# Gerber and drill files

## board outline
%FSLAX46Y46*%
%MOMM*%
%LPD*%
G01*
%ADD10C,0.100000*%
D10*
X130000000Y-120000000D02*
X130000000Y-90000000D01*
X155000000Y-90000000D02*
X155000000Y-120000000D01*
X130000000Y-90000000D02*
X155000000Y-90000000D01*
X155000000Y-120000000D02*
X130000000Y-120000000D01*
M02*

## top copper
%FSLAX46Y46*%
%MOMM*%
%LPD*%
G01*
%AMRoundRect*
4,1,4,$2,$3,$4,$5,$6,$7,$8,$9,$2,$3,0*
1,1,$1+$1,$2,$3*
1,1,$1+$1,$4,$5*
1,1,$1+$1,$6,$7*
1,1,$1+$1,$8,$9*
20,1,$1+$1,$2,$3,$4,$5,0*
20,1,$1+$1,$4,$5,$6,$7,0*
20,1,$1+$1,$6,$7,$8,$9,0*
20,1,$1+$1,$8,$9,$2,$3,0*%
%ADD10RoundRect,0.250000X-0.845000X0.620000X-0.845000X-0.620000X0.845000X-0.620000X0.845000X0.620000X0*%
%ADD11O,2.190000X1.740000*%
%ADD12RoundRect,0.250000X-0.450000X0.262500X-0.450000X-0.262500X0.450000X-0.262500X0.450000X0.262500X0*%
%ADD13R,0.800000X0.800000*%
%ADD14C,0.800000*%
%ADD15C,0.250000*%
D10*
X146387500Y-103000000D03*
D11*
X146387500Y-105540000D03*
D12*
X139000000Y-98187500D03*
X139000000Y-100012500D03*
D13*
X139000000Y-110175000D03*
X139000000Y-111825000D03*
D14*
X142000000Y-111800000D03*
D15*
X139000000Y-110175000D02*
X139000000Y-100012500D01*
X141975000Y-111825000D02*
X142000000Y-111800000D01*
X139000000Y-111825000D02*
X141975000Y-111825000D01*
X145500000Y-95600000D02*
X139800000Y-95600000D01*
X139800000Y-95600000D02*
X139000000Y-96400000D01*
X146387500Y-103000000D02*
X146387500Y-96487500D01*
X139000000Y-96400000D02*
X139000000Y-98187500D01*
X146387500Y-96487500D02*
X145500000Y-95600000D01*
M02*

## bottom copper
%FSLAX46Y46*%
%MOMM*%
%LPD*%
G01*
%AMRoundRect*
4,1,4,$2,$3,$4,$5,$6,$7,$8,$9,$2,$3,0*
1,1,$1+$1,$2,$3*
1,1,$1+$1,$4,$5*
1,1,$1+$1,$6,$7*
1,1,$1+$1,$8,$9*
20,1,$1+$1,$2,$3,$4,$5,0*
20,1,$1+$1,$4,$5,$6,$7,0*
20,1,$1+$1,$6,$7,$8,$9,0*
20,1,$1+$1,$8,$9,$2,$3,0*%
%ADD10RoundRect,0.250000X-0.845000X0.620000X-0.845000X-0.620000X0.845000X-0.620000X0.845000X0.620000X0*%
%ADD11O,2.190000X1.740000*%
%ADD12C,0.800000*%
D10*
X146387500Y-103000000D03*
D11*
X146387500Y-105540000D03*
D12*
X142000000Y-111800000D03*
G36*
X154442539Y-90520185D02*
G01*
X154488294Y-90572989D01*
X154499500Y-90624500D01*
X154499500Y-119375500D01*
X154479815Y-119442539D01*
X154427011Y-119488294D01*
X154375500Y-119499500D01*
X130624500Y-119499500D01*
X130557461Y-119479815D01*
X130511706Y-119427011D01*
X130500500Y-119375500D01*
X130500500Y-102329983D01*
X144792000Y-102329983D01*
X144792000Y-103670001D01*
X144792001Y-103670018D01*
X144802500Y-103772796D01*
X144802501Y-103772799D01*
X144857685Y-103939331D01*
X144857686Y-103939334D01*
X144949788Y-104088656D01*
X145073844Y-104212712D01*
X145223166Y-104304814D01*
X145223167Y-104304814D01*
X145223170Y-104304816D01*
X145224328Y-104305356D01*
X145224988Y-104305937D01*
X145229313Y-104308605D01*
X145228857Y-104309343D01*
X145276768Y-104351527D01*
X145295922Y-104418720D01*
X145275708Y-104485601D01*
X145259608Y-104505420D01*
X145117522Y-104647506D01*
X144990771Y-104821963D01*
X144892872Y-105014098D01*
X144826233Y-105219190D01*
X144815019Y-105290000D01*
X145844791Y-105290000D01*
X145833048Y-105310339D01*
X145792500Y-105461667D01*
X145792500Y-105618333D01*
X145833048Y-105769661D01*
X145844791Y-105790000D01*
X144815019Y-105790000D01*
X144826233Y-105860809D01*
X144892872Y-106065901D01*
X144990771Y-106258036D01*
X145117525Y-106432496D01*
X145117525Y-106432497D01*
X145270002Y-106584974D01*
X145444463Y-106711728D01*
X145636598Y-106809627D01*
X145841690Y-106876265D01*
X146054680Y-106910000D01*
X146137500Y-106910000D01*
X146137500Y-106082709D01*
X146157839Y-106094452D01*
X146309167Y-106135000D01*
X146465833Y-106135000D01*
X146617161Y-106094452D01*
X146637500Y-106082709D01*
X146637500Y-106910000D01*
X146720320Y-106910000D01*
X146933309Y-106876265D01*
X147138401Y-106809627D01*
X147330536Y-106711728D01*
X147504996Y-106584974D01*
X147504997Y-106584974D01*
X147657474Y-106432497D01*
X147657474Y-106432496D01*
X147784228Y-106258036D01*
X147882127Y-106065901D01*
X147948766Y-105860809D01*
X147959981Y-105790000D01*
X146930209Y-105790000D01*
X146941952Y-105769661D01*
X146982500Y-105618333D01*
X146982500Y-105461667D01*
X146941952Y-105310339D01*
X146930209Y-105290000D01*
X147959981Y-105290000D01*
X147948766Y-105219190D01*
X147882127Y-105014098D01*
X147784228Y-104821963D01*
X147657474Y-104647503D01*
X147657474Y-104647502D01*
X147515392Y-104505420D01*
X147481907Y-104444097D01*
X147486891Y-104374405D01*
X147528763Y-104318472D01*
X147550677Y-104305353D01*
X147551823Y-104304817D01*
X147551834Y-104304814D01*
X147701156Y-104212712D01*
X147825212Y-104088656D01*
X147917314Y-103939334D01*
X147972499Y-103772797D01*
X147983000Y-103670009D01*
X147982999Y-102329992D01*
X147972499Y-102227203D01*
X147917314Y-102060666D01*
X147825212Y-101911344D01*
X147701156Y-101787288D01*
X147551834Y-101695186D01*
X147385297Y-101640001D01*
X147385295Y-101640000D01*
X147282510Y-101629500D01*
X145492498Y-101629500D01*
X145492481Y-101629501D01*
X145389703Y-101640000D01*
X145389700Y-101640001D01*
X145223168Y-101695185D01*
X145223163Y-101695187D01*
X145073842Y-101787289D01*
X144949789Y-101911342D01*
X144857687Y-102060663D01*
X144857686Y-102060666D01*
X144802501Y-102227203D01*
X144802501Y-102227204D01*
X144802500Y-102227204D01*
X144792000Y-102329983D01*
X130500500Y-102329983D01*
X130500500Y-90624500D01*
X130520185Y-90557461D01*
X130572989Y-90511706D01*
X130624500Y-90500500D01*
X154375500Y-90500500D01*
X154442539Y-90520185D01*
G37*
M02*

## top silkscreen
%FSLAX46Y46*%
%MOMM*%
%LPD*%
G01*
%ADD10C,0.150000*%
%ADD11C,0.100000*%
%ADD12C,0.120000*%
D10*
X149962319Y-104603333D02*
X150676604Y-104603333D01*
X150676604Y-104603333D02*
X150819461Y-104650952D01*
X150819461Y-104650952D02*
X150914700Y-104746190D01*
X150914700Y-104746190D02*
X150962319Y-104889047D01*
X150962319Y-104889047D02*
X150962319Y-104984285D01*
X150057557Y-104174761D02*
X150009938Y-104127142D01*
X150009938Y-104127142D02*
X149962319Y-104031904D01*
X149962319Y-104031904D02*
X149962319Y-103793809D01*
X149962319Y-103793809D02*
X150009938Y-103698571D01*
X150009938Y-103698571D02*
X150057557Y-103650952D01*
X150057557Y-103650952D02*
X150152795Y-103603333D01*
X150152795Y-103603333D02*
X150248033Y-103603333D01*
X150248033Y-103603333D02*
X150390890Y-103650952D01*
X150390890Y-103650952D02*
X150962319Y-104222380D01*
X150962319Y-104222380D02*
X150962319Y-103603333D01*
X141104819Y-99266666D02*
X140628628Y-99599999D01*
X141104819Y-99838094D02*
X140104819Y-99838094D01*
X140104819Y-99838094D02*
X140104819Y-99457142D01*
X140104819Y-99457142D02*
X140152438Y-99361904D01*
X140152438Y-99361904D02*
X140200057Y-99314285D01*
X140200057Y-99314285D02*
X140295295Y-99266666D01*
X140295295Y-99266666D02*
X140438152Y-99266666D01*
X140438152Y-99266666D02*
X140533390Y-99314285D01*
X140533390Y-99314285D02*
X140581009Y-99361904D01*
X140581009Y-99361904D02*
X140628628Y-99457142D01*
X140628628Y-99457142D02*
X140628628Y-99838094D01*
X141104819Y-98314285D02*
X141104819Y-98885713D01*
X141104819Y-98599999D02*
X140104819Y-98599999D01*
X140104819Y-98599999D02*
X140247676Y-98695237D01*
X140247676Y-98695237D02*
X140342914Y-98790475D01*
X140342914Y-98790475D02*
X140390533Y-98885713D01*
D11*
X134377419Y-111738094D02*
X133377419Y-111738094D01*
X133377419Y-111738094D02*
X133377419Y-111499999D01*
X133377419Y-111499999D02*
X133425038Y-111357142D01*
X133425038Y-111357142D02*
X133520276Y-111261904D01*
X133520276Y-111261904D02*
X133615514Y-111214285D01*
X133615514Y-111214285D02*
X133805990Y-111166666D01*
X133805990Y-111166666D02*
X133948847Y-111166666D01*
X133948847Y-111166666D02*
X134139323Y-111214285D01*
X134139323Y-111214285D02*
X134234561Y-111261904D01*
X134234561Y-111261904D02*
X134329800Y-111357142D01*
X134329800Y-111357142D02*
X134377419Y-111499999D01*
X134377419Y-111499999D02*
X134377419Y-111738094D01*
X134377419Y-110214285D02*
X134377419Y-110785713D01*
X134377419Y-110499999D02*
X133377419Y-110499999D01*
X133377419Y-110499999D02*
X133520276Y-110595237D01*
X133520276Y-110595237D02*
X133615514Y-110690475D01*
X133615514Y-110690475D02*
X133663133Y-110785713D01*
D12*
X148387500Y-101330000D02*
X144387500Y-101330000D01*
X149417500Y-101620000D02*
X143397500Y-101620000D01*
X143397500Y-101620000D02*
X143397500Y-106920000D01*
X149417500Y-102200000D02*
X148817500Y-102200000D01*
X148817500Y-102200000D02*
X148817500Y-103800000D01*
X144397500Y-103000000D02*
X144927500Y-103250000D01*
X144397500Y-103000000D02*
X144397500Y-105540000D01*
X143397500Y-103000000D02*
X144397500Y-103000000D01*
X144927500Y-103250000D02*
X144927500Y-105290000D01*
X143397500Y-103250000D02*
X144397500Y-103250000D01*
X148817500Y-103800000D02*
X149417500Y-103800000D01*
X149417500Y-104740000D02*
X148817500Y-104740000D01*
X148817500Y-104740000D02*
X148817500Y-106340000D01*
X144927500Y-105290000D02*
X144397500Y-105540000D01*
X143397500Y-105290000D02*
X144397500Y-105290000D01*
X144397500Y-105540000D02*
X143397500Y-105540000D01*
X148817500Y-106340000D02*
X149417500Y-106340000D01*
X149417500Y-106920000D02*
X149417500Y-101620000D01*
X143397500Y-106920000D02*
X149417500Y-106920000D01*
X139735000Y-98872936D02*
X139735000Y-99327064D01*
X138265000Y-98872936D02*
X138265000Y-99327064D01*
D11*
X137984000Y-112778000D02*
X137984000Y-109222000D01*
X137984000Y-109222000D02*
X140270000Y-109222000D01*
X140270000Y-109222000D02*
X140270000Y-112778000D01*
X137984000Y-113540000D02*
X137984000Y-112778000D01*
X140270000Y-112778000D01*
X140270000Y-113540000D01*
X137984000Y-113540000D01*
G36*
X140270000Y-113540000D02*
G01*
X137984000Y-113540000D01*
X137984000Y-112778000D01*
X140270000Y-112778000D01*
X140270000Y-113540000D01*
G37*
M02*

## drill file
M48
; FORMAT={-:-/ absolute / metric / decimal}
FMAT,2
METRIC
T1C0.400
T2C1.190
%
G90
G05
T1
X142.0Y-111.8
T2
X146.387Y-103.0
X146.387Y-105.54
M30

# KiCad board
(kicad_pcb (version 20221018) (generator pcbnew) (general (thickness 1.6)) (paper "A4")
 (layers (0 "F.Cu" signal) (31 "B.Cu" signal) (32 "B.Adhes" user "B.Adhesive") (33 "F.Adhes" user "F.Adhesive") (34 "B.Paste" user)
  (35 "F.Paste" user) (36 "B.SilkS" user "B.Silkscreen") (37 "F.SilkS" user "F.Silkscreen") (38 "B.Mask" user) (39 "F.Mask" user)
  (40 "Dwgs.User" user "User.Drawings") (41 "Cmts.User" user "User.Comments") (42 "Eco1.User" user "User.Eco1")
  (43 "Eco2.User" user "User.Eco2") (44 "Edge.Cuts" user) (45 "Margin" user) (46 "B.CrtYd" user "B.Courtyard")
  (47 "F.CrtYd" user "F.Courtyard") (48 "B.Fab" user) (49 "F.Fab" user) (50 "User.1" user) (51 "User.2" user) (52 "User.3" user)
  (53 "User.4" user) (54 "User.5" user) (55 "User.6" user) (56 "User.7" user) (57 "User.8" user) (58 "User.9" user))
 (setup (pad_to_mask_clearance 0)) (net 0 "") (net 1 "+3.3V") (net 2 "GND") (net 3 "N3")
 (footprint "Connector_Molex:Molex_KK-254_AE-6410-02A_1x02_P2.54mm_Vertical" (layer "F.Cu") (at 146.3875 103 -90)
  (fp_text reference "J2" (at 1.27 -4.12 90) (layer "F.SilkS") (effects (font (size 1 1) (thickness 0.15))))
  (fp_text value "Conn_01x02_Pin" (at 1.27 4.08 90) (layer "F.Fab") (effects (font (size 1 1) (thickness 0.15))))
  (fp_line (start -1.67 -2) (end -1.67 2) (stroke (width 0.12) (type solid)) (layer "F.SilkS"))
  (fp_line (start -1.38 -3.03) (end -1.38 2.99) (stroke (width 0.12) (type solid)) (layer "F.SilkS"))
  (fp_line (start -1.38 2.99) (end 3.92 2.99) (stroke (width 0.12) (type solid)) (layer "F.SilkS"))
  (fp_line (start -0.8 -3.03) (end -0.8 -2.43) (stroke (width 0.12) (type solid)) (layer "F.SilkS"))
  (fp_line (start -0.8 -2.43) (end 0.8 -2.43) (stroke (width 0.12) (type solid)) (layer "F.SilkS"))
  (fp_line (start 0 1.99) (end 0.25 1.46) (stroke (width 0.12) (type solid)) (layer "F.SilkS"))
  (fp_line (start 0 1.99) (end 2.54 1.99) (stroke (width 0.12) (type solid)) (layer "F.SilkS"))
  (fp_line (start 0 2.99) (end 0 1.99) (stroke (width 0.12) (type solid)) (layer "F.SilkS"))
  (fp_line (start 0.25 1.46) (end 2.29 1.46) (stroke (width 0.12) (type solid)) (layer "F.SilkS"))
  (fp_line (start 0.25 2.99) (end 0.25 1.99) (stroke (width 0.12) (type solid)) (layer "F.SilkS"))
  (fp_line (start 0.8 -2.43) (end 0.8 -3.03) (stroke (width 0.12) (type solid)) (layer "F.SilkS"))
  (fp_line (start 1.74 -3.03) (end 1.74 -2.43) (stroke (width 0.12) (type solid)) (layer "F.SilkS"))
  (fp_line (start 1.74 -2.43) (end 3.34 -2.43) (stroke (width 0.12) (type solid)) (layer "F.SilkS"))
  (fp_line (start 2.29 1.46) (end 2.54 1.99) (stroke (width 0.12) (type solid)) (layer "F.SilkS"))
  (fp_line (start 2.29 2.99) (end 2.29 1.99) (stroke (width 0.12) (type solid)) (layer "F.SilkS"))
  (fp_line (start 2.54 1.99) (end 2.54 2.99) (stroke (width 0.12) (type solid)) (layer "F.SilkS"))
  (fp_line (start 3.34 -2.43) (end 3.34 -3.03) (stroke (width 0.12) (type solid)) (layer "F.SilkS"))
  (fp_line (start 3.92 -3.03) (end -1.38 -3.03) (stroke (width 0.12) (type solid)) (layer "F.SilkS"))
  (fp_line (start 3.92 2.99) (end 3.92 -3.03) (stroke (width 0.12) (type solid)) (layer "F.SilkS"))
  (pad "1" thru_hole roundrect (at 0 0 270) (size 1.74 2.19) (drill 1.19) (layers "*.Cu" "*.Mask") (roundrect_rratio 0.1436781609)
   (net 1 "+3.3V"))
  (pad "2" thru_hole oval (at 2.54 0 270) (size 1.74 2.19) (drill 1.19) (layers "*.Cu" "*.Mask") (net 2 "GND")))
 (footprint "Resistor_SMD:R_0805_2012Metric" (layer "F.Cu") (at 139 99.1 -90)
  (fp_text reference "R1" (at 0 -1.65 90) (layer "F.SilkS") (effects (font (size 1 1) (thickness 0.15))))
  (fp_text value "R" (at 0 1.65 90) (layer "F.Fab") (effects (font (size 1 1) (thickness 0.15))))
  (fp_line (start -0.227064 -0.735) (end 0.227064 -0.735) (stroke (width 0.12) (type solid)) (layer "F.SilkS"))
  (fp_line (start -0.227064 0.735) (end 0.227064 0.735) (stroke (width 0.12) (type solid)) (layer "F.SilkS"))
  (pad "1" smd roundrect (at -0.9125 0 270) (size 1.025 1.4) (layers "F.Cu" "F.Paste" "F.Mask") (roundrect_rratio 0.243902439)
   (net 1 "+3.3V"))
  (pad "2" smd roundrect (at 0.9125 0 270) (size 1.025 1.4) (layers "F.Cu" "F.Paste" "F.Mask") (roundrect_rratio 0.243902439) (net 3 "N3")))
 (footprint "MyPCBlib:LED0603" (layer "F.Cu") (at 139 111 90)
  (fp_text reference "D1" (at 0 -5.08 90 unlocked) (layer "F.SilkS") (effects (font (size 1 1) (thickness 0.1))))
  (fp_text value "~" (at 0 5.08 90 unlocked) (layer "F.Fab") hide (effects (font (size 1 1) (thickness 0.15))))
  (fp_line (start -1.778 -1.016) (end 1.778 -1.016) (stroke (width 0.1) (type default)) (layer "F.SilkS"))
  (fp_line (start 1.778 -1.016) (end 1.778 1.27) (stroke (width 0.1) (type default)) (layer "F.SilkS"))
  (fp_line (start 1.778 1.27) (end -1.778 1.27) (stroke (width 0.1) (type default)) (layer "F.SilkS"))
  (fp_poly
   (pts (xy -2.54 -1.016) (xy -1.778 -1.016) (xy -1.778 1.27) (xy -2.54 1.27)) (stroke (width 0.1) (type solid)) (fill solid)
   (layer "F.SilkS"))
  (pad "A" smd rect (at 0.825 0 90) (size 0.8 0.8) (layers "F.Cu" "F.Paste" "F.Mask") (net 3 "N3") (thermal_bridge_angle 45))
  (pad "C" smd rect (at -0.825 0 90) (size 0.8 0.8) (layers "F.Cu" "F.Paste" "F.Mask") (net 2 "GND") (thermal_bridge_angle 45)))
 (gr_line (start 130 120) (end 130 90) (stroke (width 0.1) (type default)) (layer "Edge.Cuts"))
 (gr_line (start 155 90) (end 155 120) (stroke (width 0.1) (type default)) (layer "Edge.Cuts"))
 (gr_line (start 130 90) (end 155 90) (stroke (width 0.1) (type default)) (layer "Edge.Cuts"))
 (gr_line (start 155 120) (end 130 120) (stroke (width 0.1) (type default)) (layer "Edge.Cuts"))
 (segment (start 139 110.175) (end 139 100.0125) (width 0.25) (layer "F.Cu") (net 3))
 (segment (start 141.975 111.825) (end 142 111.8) (width 0.25) (layer "F.Cu") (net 2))
 (segment (start 139 111.825) (end 141.975 111.825) (width 0.25) (layer "F.Cu") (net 2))
 (via (at 142 111.8) (size 0.8) (drill 0.4) (layers "F.Cu" "B.Cu") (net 2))
 (segment (start 145.5 95.6) (end 139.8 95.6) (width 0.25) (layer "F.Cu") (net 1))
 (segment (start 139.8 95.6) (end 139 96.4) (width 0.25) (layer "F.Cu") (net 1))
 (segment (start 146.3875 103) (end 146.3875 96.4875) (width 0.25) (layer "F.Cu") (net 1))
 (segment (start 139 96.4) (end 139 98.1875) (width 0.25) (layer "F.Cu") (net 1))
 (segment (start 146.3875 96.4875) (end 145.5 95.6) (width 0.25) (layer "F.Cu") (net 1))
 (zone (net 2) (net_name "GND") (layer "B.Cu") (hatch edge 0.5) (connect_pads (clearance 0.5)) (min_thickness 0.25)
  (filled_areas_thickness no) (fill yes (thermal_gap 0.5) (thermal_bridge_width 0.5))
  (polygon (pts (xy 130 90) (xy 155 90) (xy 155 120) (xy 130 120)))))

